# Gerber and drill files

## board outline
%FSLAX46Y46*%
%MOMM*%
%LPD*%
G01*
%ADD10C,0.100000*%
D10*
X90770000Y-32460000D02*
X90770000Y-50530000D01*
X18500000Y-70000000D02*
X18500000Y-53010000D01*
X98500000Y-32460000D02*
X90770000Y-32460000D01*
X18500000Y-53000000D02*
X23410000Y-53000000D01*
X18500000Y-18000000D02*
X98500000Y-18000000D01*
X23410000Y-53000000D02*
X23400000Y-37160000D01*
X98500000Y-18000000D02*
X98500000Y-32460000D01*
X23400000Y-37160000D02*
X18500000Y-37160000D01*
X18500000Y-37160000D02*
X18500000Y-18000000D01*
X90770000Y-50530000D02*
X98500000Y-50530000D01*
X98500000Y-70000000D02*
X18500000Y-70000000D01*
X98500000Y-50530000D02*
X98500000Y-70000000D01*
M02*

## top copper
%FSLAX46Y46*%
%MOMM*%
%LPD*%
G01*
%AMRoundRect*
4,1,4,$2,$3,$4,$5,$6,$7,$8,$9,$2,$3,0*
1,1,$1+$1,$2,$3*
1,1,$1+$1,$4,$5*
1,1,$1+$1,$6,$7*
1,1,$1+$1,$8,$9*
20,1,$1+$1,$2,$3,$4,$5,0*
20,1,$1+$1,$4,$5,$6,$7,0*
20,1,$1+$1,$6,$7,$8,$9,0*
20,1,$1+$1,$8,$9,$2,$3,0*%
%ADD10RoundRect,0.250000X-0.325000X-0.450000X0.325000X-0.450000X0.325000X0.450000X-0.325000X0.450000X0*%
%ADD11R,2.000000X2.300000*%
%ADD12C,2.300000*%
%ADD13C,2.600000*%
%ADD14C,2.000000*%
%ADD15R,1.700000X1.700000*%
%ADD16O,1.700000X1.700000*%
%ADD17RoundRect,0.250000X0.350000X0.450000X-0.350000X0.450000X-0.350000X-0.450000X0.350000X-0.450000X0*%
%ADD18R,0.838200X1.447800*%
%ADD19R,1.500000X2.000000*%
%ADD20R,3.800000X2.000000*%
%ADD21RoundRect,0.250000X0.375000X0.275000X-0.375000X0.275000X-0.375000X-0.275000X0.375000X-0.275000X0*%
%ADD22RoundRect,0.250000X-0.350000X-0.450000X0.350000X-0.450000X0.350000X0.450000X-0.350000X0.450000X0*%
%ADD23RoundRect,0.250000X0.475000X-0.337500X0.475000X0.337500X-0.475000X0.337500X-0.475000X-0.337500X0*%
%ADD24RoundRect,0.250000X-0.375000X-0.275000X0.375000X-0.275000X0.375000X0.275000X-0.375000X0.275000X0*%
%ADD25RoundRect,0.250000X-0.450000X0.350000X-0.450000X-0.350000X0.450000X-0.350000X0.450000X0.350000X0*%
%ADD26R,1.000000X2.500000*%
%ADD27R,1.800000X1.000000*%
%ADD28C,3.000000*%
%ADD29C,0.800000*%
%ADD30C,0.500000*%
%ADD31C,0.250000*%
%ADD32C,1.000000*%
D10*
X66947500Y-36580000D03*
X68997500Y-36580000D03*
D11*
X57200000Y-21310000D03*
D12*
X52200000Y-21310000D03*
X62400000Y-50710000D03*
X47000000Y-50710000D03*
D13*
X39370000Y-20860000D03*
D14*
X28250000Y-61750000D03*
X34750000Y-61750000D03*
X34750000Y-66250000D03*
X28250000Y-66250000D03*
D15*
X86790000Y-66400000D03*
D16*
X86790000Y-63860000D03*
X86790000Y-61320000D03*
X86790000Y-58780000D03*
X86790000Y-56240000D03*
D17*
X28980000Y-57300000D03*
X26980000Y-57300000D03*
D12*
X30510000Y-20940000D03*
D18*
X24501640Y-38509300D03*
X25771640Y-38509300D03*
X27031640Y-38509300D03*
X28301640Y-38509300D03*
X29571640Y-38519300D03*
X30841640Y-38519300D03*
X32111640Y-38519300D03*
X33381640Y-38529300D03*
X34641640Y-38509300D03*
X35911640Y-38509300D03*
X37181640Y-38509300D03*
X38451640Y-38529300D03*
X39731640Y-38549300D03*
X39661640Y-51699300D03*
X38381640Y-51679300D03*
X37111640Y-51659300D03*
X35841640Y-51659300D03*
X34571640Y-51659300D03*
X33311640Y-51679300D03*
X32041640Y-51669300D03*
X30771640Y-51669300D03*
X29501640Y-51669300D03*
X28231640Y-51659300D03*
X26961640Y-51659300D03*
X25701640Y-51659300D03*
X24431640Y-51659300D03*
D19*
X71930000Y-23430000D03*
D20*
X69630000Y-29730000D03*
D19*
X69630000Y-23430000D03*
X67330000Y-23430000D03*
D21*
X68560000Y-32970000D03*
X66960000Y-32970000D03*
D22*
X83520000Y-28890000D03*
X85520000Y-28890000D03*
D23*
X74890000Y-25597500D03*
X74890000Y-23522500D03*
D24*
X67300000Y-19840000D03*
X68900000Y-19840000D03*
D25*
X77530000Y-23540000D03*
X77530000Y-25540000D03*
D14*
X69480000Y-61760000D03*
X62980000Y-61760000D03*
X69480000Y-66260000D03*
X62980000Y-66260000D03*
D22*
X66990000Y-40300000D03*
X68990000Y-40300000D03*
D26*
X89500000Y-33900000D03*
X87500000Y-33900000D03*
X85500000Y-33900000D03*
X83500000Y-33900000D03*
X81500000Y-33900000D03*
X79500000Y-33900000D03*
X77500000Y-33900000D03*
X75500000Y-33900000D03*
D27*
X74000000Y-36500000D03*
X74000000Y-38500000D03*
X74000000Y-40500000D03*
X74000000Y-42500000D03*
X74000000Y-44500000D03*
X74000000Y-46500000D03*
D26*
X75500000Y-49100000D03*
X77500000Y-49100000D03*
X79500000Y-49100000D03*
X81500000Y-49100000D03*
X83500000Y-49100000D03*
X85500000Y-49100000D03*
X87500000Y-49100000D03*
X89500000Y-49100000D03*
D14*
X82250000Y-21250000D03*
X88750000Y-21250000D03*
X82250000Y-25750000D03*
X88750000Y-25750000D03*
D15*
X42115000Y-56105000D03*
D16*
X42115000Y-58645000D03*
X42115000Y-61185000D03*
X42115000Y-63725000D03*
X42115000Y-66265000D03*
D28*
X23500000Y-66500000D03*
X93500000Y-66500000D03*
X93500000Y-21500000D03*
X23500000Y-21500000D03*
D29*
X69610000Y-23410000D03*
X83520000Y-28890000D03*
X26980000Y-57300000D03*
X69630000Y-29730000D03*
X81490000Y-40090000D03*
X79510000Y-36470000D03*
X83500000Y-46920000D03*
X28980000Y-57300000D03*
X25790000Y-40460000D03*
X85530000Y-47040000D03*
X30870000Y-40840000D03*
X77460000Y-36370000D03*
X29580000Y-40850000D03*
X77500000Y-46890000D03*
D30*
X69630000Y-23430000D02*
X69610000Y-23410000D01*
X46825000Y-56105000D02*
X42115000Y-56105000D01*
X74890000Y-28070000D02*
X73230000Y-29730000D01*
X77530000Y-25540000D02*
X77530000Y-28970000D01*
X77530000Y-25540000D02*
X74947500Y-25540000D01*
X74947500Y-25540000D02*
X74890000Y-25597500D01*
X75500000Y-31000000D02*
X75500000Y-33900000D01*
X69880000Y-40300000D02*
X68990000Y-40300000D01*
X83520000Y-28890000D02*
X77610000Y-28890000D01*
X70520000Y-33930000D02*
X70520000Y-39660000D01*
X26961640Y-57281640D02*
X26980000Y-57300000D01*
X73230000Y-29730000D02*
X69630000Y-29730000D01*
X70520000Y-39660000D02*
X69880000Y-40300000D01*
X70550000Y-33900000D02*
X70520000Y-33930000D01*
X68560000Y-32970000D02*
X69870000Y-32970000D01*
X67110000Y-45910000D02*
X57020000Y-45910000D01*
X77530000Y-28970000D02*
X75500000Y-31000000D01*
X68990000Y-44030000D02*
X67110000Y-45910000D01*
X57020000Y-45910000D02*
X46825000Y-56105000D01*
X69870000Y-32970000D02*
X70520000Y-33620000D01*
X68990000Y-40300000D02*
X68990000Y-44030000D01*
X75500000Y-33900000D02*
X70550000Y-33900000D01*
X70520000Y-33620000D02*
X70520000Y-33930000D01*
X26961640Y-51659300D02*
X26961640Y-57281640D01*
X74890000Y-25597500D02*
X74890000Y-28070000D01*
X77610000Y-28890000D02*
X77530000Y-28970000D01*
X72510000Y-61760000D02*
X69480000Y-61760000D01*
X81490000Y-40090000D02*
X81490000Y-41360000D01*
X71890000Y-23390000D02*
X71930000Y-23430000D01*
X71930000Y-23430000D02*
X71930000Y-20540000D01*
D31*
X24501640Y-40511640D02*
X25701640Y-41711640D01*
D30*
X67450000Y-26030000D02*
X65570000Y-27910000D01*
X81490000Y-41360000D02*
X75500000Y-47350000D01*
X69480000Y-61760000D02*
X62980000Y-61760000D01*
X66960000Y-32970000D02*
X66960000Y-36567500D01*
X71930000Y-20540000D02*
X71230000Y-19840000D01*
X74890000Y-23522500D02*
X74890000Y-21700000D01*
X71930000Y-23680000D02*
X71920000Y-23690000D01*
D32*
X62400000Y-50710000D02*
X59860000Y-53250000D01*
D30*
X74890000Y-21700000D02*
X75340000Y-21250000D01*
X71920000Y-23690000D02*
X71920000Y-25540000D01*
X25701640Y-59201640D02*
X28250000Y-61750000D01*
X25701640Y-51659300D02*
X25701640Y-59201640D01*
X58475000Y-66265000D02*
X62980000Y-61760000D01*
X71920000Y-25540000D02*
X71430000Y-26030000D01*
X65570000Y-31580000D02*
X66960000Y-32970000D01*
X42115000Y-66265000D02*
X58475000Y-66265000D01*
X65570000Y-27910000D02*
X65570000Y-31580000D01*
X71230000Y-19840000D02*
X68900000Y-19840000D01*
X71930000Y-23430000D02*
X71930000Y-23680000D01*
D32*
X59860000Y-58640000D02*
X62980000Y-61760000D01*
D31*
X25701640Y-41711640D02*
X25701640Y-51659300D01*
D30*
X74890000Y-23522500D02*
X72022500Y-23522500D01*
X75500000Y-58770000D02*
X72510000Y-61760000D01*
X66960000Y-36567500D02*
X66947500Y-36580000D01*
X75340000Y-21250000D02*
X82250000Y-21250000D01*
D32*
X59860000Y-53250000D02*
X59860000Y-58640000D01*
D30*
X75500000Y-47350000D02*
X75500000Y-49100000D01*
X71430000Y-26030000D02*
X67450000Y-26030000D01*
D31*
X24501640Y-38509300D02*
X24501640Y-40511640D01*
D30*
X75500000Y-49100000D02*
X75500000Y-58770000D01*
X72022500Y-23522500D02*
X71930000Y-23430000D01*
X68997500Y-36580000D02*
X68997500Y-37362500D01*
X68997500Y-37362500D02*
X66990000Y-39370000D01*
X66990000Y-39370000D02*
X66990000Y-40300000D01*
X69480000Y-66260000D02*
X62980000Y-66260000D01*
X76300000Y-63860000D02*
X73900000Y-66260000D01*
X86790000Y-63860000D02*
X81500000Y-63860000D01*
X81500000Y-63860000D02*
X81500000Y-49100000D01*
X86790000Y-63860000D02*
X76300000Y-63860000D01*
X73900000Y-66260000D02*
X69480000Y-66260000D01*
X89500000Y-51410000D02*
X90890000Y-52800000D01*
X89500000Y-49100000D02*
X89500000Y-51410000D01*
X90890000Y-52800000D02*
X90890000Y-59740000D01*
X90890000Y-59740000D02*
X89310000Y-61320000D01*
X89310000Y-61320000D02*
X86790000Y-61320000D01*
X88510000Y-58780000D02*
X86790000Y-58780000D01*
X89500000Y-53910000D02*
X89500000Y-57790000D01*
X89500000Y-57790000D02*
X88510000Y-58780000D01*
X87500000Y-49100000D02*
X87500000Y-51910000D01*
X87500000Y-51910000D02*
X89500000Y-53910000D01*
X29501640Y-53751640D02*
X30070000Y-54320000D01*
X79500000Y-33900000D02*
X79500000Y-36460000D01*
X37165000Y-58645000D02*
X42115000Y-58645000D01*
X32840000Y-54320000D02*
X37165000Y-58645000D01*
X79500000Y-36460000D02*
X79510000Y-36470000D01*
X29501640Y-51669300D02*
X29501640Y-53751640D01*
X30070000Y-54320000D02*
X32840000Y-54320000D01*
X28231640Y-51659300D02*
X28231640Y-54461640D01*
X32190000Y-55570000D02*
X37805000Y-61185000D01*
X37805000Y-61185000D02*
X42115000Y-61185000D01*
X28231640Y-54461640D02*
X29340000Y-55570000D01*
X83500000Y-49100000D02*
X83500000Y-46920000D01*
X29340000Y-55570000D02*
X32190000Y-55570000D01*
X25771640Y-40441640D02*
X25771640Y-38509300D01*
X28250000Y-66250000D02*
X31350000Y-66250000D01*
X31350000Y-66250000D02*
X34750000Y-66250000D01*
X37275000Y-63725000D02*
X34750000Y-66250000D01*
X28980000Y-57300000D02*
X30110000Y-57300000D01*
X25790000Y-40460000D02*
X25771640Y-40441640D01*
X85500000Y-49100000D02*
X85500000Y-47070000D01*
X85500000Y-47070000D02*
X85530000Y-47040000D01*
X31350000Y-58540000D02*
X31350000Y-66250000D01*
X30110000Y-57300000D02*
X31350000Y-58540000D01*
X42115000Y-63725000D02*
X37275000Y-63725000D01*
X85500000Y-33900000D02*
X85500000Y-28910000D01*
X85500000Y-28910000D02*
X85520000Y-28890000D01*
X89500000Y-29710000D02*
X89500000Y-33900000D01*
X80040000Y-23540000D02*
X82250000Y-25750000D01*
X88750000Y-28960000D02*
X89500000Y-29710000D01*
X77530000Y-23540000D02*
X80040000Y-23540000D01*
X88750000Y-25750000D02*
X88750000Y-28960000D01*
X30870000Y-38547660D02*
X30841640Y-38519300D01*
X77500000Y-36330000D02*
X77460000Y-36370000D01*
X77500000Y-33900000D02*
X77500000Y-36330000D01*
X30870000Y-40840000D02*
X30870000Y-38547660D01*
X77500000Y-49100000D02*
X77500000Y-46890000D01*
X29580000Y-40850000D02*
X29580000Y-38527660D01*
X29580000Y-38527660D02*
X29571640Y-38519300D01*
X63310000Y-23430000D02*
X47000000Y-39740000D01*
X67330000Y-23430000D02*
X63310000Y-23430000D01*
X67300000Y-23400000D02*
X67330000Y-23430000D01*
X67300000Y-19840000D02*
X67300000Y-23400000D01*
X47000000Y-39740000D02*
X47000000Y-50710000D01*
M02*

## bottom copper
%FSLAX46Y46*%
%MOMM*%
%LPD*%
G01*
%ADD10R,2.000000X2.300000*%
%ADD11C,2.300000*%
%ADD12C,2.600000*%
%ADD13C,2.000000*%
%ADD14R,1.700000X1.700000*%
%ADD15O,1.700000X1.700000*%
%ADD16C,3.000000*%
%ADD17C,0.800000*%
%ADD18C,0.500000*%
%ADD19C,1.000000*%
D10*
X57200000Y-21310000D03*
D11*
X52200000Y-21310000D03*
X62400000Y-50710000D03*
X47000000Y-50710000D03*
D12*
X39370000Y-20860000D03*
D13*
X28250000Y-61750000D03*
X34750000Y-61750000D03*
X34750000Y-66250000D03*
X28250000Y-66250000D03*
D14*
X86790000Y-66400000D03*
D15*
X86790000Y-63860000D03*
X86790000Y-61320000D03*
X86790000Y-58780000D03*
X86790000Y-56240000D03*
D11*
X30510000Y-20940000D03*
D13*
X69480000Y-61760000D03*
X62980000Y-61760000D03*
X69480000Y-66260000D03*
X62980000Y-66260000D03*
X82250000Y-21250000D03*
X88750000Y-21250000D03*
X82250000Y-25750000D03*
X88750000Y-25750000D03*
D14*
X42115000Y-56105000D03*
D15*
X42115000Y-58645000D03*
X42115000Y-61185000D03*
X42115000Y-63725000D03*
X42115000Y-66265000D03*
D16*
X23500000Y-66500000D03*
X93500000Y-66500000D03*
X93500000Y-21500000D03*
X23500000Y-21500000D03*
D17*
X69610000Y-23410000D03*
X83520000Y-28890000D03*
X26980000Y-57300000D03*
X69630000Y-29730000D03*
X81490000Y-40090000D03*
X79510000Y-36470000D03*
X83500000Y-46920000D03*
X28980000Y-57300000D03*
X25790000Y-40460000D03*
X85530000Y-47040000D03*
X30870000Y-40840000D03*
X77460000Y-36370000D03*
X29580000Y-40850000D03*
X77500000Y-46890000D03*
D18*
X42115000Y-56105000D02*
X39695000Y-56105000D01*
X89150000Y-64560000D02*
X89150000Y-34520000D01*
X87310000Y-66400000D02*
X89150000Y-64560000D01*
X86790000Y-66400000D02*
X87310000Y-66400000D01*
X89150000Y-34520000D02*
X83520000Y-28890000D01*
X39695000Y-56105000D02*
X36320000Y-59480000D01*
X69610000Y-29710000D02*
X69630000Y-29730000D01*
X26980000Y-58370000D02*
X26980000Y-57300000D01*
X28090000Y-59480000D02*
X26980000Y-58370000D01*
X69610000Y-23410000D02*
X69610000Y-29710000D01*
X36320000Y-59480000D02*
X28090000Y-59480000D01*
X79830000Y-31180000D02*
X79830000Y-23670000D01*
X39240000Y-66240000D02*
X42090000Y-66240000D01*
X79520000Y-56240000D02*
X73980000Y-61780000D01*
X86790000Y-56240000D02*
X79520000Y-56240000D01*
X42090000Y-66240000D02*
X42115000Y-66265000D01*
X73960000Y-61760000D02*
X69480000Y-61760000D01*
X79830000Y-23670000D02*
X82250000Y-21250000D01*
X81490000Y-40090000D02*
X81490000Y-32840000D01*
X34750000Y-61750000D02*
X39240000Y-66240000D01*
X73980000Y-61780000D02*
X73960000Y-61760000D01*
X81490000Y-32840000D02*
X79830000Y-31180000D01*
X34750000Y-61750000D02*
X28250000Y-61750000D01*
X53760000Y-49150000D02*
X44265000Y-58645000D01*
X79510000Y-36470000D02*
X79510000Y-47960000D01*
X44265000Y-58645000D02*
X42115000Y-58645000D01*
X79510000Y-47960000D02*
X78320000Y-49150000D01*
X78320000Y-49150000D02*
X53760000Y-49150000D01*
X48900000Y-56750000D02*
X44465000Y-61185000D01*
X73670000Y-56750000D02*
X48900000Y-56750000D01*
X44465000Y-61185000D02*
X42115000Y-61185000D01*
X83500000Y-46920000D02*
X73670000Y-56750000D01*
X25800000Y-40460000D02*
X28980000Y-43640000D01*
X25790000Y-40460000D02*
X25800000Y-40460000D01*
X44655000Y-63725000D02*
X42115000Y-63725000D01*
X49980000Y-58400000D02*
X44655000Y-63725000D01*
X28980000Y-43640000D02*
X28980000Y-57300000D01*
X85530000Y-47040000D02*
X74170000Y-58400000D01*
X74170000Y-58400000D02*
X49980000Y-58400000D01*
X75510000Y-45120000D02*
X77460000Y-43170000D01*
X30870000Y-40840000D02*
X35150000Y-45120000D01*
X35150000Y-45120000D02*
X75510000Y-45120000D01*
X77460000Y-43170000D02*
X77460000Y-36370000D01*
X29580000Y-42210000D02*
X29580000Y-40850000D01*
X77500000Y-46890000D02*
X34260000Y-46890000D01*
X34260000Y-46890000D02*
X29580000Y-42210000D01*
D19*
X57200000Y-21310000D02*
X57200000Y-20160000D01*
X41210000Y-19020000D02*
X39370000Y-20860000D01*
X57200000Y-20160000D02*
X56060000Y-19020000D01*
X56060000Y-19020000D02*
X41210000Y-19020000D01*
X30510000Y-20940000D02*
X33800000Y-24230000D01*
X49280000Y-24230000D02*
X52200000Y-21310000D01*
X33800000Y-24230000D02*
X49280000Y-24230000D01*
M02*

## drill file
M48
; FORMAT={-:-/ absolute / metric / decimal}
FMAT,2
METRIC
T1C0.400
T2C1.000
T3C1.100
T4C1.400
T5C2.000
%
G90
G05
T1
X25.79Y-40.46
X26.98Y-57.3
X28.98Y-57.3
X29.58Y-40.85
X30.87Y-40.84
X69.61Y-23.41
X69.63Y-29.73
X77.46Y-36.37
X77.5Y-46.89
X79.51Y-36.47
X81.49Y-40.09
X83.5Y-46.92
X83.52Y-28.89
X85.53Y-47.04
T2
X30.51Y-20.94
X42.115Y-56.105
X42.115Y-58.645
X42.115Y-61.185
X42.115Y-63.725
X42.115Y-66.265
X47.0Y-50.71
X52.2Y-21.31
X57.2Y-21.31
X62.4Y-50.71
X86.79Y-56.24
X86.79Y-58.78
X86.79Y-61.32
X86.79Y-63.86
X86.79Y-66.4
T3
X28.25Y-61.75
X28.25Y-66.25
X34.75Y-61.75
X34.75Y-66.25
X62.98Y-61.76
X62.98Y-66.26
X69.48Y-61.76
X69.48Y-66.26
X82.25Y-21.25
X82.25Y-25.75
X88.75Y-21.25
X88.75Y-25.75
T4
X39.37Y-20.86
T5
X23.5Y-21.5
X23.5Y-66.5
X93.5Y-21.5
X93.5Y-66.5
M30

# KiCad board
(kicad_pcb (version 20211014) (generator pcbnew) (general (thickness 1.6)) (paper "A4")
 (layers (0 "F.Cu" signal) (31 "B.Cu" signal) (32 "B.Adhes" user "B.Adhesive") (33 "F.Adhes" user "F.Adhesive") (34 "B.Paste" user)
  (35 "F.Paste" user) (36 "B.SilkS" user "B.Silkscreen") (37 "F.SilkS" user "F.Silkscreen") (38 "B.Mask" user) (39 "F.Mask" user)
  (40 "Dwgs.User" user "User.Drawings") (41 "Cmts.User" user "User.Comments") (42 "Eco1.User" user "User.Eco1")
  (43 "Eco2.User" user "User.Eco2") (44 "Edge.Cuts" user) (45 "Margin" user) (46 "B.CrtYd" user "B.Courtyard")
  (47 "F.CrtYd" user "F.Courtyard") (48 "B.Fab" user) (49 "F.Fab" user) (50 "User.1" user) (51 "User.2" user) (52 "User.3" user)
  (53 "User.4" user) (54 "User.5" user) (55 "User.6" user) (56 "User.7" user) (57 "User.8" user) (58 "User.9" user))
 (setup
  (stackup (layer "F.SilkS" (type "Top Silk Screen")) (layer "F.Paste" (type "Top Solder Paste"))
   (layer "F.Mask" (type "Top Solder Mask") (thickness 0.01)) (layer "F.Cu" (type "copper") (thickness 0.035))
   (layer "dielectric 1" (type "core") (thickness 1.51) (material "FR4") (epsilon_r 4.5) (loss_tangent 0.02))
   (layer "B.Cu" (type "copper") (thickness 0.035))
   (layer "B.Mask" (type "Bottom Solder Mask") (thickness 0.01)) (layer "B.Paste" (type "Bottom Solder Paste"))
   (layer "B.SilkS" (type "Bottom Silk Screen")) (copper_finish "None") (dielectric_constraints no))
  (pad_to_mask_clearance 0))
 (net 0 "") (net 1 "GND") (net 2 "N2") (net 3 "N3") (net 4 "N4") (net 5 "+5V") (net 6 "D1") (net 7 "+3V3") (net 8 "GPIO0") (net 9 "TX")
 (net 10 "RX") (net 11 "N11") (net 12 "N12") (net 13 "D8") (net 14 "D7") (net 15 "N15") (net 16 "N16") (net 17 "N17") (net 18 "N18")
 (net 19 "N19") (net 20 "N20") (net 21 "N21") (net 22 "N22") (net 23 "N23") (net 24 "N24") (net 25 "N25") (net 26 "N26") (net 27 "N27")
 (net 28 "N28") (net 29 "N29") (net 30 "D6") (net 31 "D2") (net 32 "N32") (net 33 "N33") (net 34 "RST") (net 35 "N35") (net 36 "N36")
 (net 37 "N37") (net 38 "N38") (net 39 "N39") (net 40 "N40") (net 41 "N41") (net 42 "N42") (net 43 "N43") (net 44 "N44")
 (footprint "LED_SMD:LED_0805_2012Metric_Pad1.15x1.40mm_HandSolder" (layer "F.Cu") (at 67.9725 36.58)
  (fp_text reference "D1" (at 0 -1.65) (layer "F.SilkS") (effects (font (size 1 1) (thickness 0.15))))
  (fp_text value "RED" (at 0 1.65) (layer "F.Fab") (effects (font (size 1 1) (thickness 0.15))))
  (pad "1" smd roundrect (at -1.025 0) (size 1.15 1.4) (layers "F.Cu" "F.Paste" "F.Mask") (roundrect_rratio 0.217391) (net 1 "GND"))
  (pad "2" smd roundrect (at 1.025 0) (size 1.15 1.4) (layers "F.Cu" "F.Paste" "F.Mask") (roundrect_rratio 0.217391) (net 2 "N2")))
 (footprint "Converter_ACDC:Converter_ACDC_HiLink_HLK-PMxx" (layer "F.Cu") (at 57.2 21.31 -90)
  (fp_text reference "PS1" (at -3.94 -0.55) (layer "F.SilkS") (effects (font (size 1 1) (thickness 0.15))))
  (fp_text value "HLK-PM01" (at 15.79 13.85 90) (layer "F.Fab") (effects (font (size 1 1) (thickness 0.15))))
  (pad "1" thru_hole rect (at 0 0 270) (size 2.3 2) (drill 1) (layers *.Cu *.Mask) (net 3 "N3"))
  (pad "2" thru_hole circle (at 0 5 270) (size 2.3 2.3) (drill 1) (layers *.Cu *.Mask) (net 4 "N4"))
  (pad "3" thru_hole circle (at 29.4 -5.2 270) (size 2.3 2.3) (drill 1) (layers *.Cu *.Mask) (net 1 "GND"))
  (pad "4" thru_hole circle (at 29.4 10.2 270) (size 2.3 2.3) (drill 1) (layers *.Cu *.Mask) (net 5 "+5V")))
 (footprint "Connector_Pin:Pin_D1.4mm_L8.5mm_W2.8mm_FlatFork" (layer "F.Cu") (at 39.37 20.86)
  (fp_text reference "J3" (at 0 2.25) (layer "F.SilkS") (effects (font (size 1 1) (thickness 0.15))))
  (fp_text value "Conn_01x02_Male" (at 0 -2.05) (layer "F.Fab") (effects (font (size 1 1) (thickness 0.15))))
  (pad "1" thru_hole circle (at 0 0) (size 2.6 2.6) (drill 1.4) (layers *.Cu *.Mask) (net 3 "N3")))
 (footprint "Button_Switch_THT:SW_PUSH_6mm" (layer "F.Cu") (at 28.25 61.75)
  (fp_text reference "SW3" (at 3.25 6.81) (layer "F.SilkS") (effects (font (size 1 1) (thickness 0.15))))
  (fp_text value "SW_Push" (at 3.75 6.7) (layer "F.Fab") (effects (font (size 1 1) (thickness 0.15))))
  (pad "1" thru_hole circle (at 0 0 90) (size 2 2) (drill 1.1) (layers *.Cu *.Mask) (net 1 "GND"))
  (pad "1" thru_hole circle (at 6.5 0 90) (size 2 2) (drill 1.1) (layers *.Cu *.Mask) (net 1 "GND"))
  (pad "2" thru_hole circle (at 6.5 4.5 90) (size 2 2) (drill 1.1) (layers *.Cu *.Mask) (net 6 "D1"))
  (pad "2" thru_hole circle (at 0 4.5 90) (size 2 2) (drill 1.1) (layers *.Cu *.Mask) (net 6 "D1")))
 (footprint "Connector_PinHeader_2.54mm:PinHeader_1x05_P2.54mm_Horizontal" (layer "F.Cu") (at 86.79 66.4 180)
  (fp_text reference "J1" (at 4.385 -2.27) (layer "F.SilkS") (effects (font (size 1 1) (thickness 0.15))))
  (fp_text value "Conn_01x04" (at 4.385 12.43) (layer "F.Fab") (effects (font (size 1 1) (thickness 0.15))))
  (pad "1" thru_hole rect (at 0 0 180) (size 1.7 1.7) (drill 1) (layers *.Cu *.Mask) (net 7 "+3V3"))
  (pad "2" thru_hole oval (at 0 2.54 180) (size 1.7 1.7) (drill 1) (layers *.Cu *.Mask) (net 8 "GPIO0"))
  (pad "3" thru_hole oval (at 0 5.08 180) (size 1.7 1.7) (drill 1) (layers *.Cu *.Mask) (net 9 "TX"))
  (pad "4" thru_hole oval (at 0 7.62 180) (size 1.7 1.7) (drill 1) (layers *.Cu *.Mask) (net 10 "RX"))
  (pad "5" thru_hole oval (at 0 10.16 180) (size 1.7 1.7) (drill 1) (layers *.Cu *.Mask) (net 1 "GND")))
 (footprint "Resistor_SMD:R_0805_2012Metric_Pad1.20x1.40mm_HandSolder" (layer "F.Cu") (at 27.98 57.3 180)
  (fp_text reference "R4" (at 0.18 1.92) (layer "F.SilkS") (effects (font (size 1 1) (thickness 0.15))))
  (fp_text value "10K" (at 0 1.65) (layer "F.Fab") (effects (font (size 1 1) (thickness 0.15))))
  (pad "1" smd roundrect (at -1 0 180) (size 1.2 1.4) (layers "F.Cu" "F.Paste" "F.Mask") (roundrect_rratio 0.208333) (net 6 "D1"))
  (pad "2" smd roundrect (at 1 0 180) (size 1.2 1.4) (layers "F.Cu" "F.Paste" "F.Mask") (roundrect_rratio 0.208333) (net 7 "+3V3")))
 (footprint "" (layer "F.Cu") (at 30.51 20.94)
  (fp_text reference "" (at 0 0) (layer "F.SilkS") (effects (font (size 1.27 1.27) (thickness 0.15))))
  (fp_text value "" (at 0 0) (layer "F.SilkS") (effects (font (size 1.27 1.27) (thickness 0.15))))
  (pad "2" thru_hole circle (at 0 0 270) (size 2.3 2.3) (drill 1) (layers *.Cu *.Mask) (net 4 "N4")))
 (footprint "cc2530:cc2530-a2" (layer "F.Cu") (at 29.09396 45.0625 90)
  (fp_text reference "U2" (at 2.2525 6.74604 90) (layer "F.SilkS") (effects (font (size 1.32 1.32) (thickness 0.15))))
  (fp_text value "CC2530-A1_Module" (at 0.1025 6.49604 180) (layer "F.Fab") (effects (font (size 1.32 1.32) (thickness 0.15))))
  (pad "1" smd rect (at 6.5532 -4.59232 90) (size 1.4478 0.8382) (layers "F.Cu" "F.Paste" "F.Mask") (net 1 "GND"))
  (pad "2" smd rect (at 6.5532 -3.32232 90) (size 1.4478 0.8382) (layers "F.Cu" "F.Paste" "F.Mask") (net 6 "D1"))
  (pad "3" smd rect (at 6.5532 -2.06232 90) (size 1.4478 0.8382) (layers "F.Cu" "F.Paste" "F.Mask") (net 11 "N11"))
  (pad "4" smd rect (at 6.5532 -0.79232 90) (size 1.4478 0.8382) (layers "F.Cu" "F.Paste" "F.Mask") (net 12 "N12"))
  (pad "5" smd rect (at 6.5432 0.47768 90) (size 1.4478 0.8382) (layers "F.Cu" "F.Paste" "F.Mask") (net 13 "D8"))
  (pad "6" smd rect (at 6.5432 1.74768 90) (size 1.4478 0.8382) (layers "F.Cu" "F.Paste" "F.Mask") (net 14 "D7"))
  (pad "7" smd rect (at 6.5432 3.01768 90) (size 1.4478 0.8382) (layers "F.Cu" "F.Paste" "F.Mask") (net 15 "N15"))
  (pad "8" smd rect (at 6.5332 4.28768 90) (size 1.4478 0.8382) (layers "F.Cu" "F.Paste" "F.Mask") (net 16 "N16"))
  (pad "9" smd rect (at 6.5532 5.54768 90) (size 1.4478 0.8382) (layers "F.Cu" "F.Paste" "F.Mask") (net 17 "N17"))
  (pad "10" smd rect (at 6.5532 6.81768 90) (size 1.4478 0.8382) (layers "F.Cu" "F.Paste" "F.Mask") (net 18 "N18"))
  (pad "11" smd rect (at 6.5532 8.08768 90) (size 1.4478 0.8382) (layers "F.Cu" "F.Paste" "F.Mask") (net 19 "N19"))
  (pad "12" smd rect (at 6.5332 9.35768 90) (size 1.4478 0.8382) (layers "F.Cu" "F.Paste" "F.Mask") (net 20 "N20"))
  (pad "13" smd rect (at 6.5132 10.63768 270) (size 1.4478 0.8382) (layers "F.Cu" "F.Paste" "F.Mask") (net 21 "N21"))
  (pad "14" smd rect (at -6.6368 10.56768 270) (size 1.4478 0.8382) (layers "F.Cu" "F.Paste" "F.Mask") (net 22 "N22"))
  (pad "15" smd rect (at -6.6168 9.28768 90) (size 1.4478 0.8382) (layers "F.Cu" "F.Paste" "F.Mask") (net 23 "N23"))
  (pad "16" smd rect (at -6.5968 8.01768 90) (size 1.4478 0.8382) (layers "F.Cu" "F.Paste" "F.Mask") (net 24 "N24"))
  (pad "17" smd rect (at -6.5968 6.74768 90) (size 1.4478 0.8382) (layers "F.Cu" "F.Paste" "F.Mask") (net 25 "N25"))
  (pad "18" smd rect (at -6.5968 5.47768 90) (size 1.4478 0.8382) (layers "F.Cu" "F.Paste" "F.Mask") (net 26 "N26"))
  (pad "19" smd rect (at -6.6168 4.21768 90) (size 1.4478 0.8382) (layers "F.Cu" "F.Paste" "F.Mask") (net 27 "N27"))
  (pad "20" smd rect (at -6.6068 2.94768 90) (size 1.4478 0.8382) (layers "F.Cu" "F.Paste" "F.Mask") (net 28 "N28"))
  (pad "21" smd rect (at -6.6068 1.67768 90) (size 1.4478 0.8382) (layers "F.Cu" "F.Paste" "F.Mask") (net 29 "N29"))
  (pad "22" smd rect (at -6.6068 0.40768 90) (size 1.4478 0.8382) (layers "F.Cu" "F.Paste" "F.Mask") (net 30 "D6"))
  (pad "23" smd rect (at -6.5968 -0.86232 90) (size 1.4478 0.8382) (layers "F.Cu" "F.Paste" "F.Mask") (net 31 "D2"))
  (pad "24" smd rect (at -6.5968 -2.13232 90) (size 1.4478 0.8382) (layers "F.Cu" "F.Paste" "F.Mask") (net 7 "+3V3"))
  (pad "25" smd rect (at -6.5968 -3.39232 90) (size 1.4478 0.8382) (layers "F.Cu" "F.Paste" "F.Mask") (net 1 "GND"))
  (pad "26" smd rect (at -6.5968 -4.66232 90) (size 1.4478 0.8382) (layers "F.Cu" "F.Paste" "F.Mask") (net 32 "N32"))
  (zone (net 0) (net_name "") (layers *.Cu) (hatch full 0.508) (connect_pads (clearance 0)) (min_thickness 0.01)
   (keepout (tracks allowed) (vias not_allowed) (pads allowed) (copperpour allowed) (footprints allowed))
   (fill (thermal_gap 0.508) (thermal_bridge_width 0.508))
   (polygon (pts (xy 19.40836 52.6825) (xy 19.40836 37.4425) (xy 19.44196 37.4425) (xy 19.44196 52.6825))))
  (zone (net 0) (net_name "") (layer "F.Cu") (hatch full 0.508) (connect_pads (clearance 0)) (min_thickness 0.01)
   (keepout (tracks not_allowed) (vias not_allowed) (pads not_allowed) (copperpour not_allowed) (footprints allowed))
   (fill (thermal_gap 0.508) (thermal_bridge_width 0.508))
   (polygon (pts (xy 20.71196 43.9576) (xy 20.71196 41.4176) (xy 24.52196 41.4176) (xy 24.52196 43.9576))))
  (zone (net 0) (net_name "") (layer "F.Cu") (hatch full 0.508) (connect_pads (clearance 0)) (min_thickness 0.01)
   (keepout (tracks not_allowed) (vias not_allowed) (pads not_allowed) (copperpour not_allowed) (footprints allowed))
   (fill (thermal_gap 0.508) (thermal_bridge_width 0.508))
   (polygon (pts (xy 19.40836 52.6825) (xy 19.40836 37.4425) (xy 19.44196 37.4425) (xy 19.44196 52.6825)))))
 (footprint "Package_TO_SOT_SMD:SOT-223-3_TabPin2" (layer "F.Cu") (at 69.63 26.58 -90)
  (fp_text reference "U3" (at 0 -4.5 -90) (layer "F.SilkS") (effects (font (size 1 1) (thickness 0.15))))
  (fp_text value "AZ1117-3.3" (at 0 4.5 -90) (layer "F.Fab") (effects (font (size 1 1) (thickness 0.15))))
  (pad "1" smd rect (at -3.15 -2.3 270) (size 2 1.5) (layers "F.Cu" "F.Paste" "F.Mask") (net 1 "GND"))
  (pad "2" smd rect (at 3.15 0 270) (size 2 3.8) (layers "F.Cu" "F.Paste" "F.Mask") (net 7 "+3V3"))
  (pad "2" smd rect (at -3.15 0 270) (size 2 1.5) (layers "F.Cu" "F.Paste" "F.Mask") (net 7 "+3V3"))
  (pad "3" smd rect (at -3.15 2.3 270) (size 2 1.5) (layers "F.Cu" "F.Paste" "F.Mask") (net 5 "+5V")))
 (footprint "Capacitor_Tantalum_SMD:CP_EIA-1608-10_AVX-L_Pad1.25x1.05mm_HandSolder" (layer "F.Cu") (at 67.76 32.97 180)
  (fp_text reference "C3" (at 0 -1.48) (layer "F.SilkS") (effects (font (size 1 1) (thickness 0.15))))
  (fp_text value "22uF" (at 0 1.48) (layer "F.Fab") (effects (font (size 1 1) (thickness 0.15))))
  (pad "1" smd roundrect (at -0.8 0 180) (size 1.25 1.05) (layers "F.Cu" "F.Paste" "F.Mask") (roundrect_rratio 0.238095) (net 7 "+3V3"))
  (pad "2" smd roundrect (at 0.8 0 180) (size 1.25 1.05) (layers "F.Cu" "F.Paste" "F.Mask") (roundrect_rratio 0.238095) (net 1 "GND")))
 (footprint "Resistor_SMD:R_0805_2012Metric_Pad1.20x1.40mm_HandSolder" (layer "F.Cu") (at 84.52 28.89)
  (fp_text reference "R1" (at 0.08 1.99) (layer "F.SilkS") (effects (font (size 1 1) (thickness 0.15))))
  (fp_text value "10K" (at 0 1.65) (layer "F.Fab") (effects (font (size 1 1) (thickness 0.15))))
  (pad "1" smd roundrect (at -1 0) (size 1.2 1.4) (layers "F.Cu" "F.Paste" "F.Mask") (roundrect_rratio 0.208333) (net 7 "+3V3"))
  (pad "2" smd roundrect (at 1 0) (size 1.2 1.4) (layers "F.Cu" "F.Paste" "F.Mask") (roundrect_rratio 0.208333) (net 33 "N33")))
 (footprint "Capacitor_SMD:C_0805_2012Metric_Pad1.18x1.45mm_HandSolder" (layer "F.Cu") (at 74.89 24.56 90)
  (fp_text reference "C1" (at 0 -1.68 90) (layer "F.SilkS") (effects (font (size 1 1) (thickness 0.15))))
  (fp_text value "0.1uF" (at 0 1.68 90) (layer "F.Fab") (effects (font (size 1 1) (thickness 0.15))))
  (pad "1" smd roundrect (at -1.0375 0 90) (size 1.175 1.45) (layers "F.Cu" "F.Paste" "F.Mask") (roundrect_rratio 0.212766) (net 7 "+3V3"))
  (pad "2" smd roundrect (at 1.0375 0 90) (size 1.175 1.45) (layers "F.Cu" "F.Paste" "F.Mask") (roundrect_rratio 0.212766) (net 1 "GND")))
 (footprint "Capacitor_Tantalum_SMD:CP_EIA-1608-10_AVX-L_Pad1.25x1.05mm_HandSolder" (layer "F.Cu") (at 68.1 19.84)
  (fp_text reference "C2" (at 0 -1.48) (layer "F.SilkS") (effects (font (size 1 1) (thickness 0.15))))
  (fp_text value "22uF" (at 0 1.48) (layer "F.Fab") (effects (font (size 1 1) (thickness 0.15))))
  (pad "1" smd roundrect (at -0.8 0) (size 1.25 1.05) (layers "F.Cu" "F.Paste" "F.Mask") (roundrect_rratio 0.238095) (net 5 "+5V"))
  (pad "2" smd roundrect (at 0.8 0) (size 1.25 1.05) (layers "F.Cu" "F.Paste" "F.Mask") (roundrect_rratio 0.238095) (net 1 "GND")))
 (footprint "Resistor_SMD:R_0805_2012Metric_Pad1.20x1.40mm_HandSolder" (layer "F.Cu") (at 77.53 24.54 -90)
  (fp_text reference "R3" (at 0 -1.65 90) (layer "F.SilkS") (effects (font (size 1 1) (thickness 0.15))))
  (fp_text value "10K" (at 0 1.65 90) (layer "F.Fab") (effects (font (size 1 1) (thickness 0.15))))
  (pad "1" smd roundrect (at -1 0 270) (size 1.2 1.4) (layers "F.Cu" "F.Paste" "F.Mask") (roundrect_rratio 0.208333) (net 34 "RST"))
  (pad "2" smd roundrect (at 1 0 270) (size 1.2 1.4) (layers "F.Cu" "F.Paste" "F.Mask") (roundrect_rratio 0.208333) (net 7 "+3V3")))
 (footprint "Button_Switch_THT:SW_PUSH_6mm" (layer "F.Cu") (at 62.98 61.76)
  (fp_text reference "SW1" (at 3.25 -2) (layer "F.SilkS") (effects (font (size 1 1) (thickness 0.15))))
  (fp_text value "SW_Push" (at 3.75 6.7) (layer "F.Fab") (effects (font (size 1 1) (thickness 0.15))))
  (pad "1" thru_hole circle (at 6.5 0 90) (size 2 2) (drill 1.1) (layers *.Cu *.Mask) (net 1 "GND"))
  (pad "1" thru_hole circle (at 0 0 90) (size 2 2) (drill 1.1) (layers *.Cu *.Mask) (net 1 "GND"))
  (pad "2" thru_hole circle (at 6.5 4.5 90) (size 2 2) (drill 1.1) (layers *.Cu *.Mask) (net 8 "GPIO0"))
  (pad "2" thru_hole circle (at 0 4.5 90) (size 2 2) (drill 1.1) (layers *.Cu *.Mask) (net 8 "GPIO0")))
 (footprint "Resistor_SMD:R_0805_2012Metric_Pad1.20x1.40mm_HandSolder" (layer "F.Cu") (at 67.99 40.3)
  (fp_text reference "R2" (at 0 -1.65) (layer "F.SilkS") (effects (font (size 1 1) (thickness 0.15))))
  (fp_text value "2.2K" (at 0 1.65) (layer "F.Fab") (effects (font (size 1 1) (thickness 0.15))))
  (pad "1" smd roundrect (at -1 0) (size 1.2 1.4) (layers "F.Cu" "F.Paste" "F.Mask") (roundrect_rratio 0.208333) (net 2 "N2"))
  (pad "2" smd roundrect (at 1 0) (size 1.2 1.4) (layers "F.Cu" "F.Paste" "F.Mask") (roundrect_rratio 0.208333) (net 7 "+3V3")))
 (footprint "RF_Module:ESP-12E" (layer "F.Cu") (at 86 41.5 -90)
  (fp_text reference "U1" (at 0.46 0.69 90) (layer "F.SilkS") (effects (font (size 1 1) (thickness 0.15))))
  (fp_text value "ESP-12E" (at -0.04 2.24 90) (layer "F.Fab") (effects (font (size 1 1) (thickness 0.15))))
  (pad "1" smd rect (at -7.6 -3.5 270) (size 2.5 1) (layers "F.Cu" "F.Paste" "F.Mask") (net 34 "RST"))
  (pad "2" smd rect (at -7.6 -1.5 270) (size 2.5 1) (layers "F.Cu" "F.Paste" "F.Mask") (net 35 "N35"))
  (pad "3" smd rect (at -7.6 0.5 270) (size 2.5 1) (layers "F.Cu" "F.Paste" "F.Mask") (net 33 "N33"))
  (pad "4" smd rect (at -7.6 2.5 270) (size 2.5 1) (layers "F.Cu" "F.Paste" "F.Mask") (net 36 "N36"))
  (pad "5" smd rect (at -7.6 4.5 270) (size 2.5 1) (layers "F.Cu" "F.Paste" "F.Mask") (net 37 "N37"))
  (pad "6" smd rect (at -7.6 6.5 270) (size 2.5 1) (layers "F.Cu" "F.Paste" "F.Mask") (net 30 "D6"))
  (pad "7" smd rect (at -7.6 8.5 270) (size 2.5 1) (layers "F.Cu" "F.Paste" "F.Mask") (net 14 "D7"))
  (pad "8" smd rect (at -7.6 10.5 270) (size 2.5 1) (layers "F.Cu" "F.Paste" "F.Mask") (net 7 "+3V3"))
  (pad "9" smd rect (at -5 12 270) (size 1 1.8) (layers "F.Cu" "F.Paste" "F.Mask") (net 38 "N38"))
  (pad "10" smd rect (at -3 12 270) (size 1 1.8) (layers "F.Cu" "F.Paste" "F.Mask") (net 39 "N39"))
  (pad "11" smd rect (at -1 12 270) (size 1 1.8) (layers "F.Cu" "F.Paste" "F.Mask") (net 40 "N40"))
  (pad "12" smd rect (at 1 12 270) (size 1 1.8) (layers "F.Cu" "F.Paste" "F.Mask") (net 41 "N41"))
  (pad "13" smd rect (at 3 12 270) (size 1 1.8) (layers "F.Cu" "F.Paste" "F.Mask") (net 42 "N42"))
  (pad "14" smd rect (at 5 12 270) (size 1 1.8) (layers "F.Cu" "F.Paste" "F.Mask") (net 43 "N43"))
  (pad "15" smd rect (at 7.6 10.5 270) (size 2.5 1) (layers "F.Cu" "F.Paste" "F.Mask") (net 1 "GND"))
  (pad "16" smd rect (at 7.6 8.5 270) (size 2.5 1) (layers "F.Cu" "F.Paste" "F.Mask") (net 13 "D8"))
  (pad "17" smd rect (at 7.6 6.5 270) (size 2.5 1) (layers "F.Cu" "F.Paste" "F.Mask") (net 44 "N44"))
  (pad "18" smd rect (at 7.6 4.5 270) (size 2.5 1) (layers "F.Cu" "F.Paste" "F.Mask") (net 8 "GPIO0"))
  (pad "19" smd rect (at 7.6 2.5 270) (size 2.5 1) (layers "F.Cu" "F.Paste" "F.Mask") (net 31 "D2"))
  (pad "20" smd rect (at 7.6 0.5 270) (size 2.5 1) (layers "F.Cu" "F.Paste" "F.Mask") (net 6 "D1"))
  (pad "21" smd rect (at 7.6 -1.5 270) (size 2.5 1) (layers "F.Cu" "F.Paste" "F.Mask") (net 10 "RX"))
  (pad "22" smd rect (at 7.6 -3.5 270) (size 2.5 1) (layers "F.Cu" "F.Paste" "F.Mask") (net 9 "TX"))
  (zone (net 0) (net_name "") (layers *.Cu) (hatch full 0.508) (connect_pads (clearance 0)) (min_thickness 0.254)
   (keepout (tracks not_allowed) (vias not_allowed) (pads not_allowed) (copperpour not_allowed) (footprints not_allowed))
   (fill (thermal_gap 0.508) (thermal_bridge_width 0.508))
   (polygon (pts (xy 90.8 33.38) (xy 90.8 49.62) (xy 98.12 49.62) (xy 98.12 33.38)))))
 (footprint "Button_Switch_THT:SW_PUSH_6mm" (layer "F.Cu") (at 82.25 21.25)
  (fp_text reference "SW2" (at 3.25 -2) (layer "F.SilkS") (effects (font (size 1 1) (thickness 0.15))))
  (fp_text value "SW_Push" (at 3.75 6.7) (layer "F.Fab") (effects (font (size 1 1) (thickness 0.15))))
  (pad "1" thru_hole circle (at 0 0 90) (size 2 2) (drill 1.1) (layers *.Cu *.Mask) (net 1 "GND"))
  (pad "1" thru_hole circle (at 6.5 0 90) (size 2 2) (drill 1.1) (layers *.Cu *.Mask) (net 1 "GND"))
  (pad "2" thru_hole circle (at 0 4.5 90) (size 2 2) (drill 1.1) (layers *.Cu *.Mask) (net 34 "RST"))
  (pad "2" thru_hole circle (at 6.5 4.5 90) (size 2 2) (drill 1.1) (layers *.Cu *.Mask) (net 34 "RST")))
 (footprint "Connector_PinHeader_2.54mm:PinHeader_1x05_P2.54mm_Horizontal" (layer "F.Cu") (at 42.115 56.105)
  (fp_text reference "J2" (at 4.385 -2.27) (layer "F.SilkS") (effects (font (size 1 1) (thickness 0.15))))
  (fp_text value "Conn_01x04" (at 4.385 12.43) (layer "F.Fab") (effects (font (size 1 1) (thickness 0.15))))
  (pad "1" thru_hole rect (at 0 0) (size 1.7 1.7) (drill 1) (layers *.Cu *.Mask) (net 7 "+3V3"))
  (pad "2" thru_hole oval (at 0 2.54) (size 1.7 1.7) (drill 1) (layers *.Cu *.Mask) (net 30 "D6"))
  (pad "3" thru_hole oval (at 0 5.08) (size 1.7 1.7) (drill 1) (layers *.Cu *.Mask) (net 31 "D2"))
  (pad "4" thru_hole oval (at 0 7.62) (size 1.7 1.7) (drill 1) (layers *.Cu *.Mask) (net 6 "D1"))
  (pad "5" thru_hole oval (at 0 10.16) (size 1.7 1.7) (drill 1) (layers *.Cu *.Mask) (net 1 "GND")))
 (gr_line (start 90.77 32.46) (end 90.77 50.53) (layer "Edge.Cuts") (width 0.1))
 (gr_line (start 18.5 70) (end 18.5 53.01) (layer "Edge.Cuts") (width 0.1))
 (gr_line (start 98.5 32.46) (end 90.77 32.46) (layer "Edge.Cuts") (width 0.1))
 (gr_line (start 18.5 53) (end 23.41 53) (layer "Edge.Cuts") (width 0.1))
 (gr_line (start 18.5 18) (end 98.5 18) (layer "Edge.Cuts") (width 0.1))
 (gr_line (start 23.41 53) (end 23.4 37.16) (layer "Edge.Cuts") (width 0.1))
 (gr_line (start 98.5 18) (end 98.5 32.46) (layer "Edge.Cuts") (width 0.1))
 (gr_line (start 23.4 37.16) (end 18.5 37.16) (layer "Edge.Cuts") (width 0.1))
 (gr_line (start 18.5 37.16) (end 18.5 18) (layer "Edge.Cuts") (width 0.1))
 (gr_line (start 90.77 50.53) (end 98.5 50.53) (layer "Edge.Cuts") (width 0.1))
 (gr_line (start 98.5 70) (end 18.5 70) (layer "Edge.Cuts") (width 0.1))
 (gr_line (start 98.5 50.53) (end 98.5 70) (layer "Edge.Cuts") (width 0.1))
 (via (at 23.5 66.5) (size 3) (drill 2) (layers "F.Cu" "B.Cu") (free) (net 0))
 (via (at 93.5 66.5) (size 3) (drill 2) (layers "F.Cu" "B.Cu") (free) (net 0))
 (via (at 93.5 21.5) (size 3) (drill 2) (layers "F.Cu" "B.Cu") (free) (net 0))
 (via (at 23.5 21.5) (size 3) (drill 2) (layers "F.Cu" "B.Cu") (free) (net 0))
 (segment (start 69.63 23.43) (end 69.61 23.41) (width 0.5) (layer "F.Cu") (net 7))
 (segment (start 46.825 56.105) (end 42.115 56.105) (width 0.5) (layer "F.Cu") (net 7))
 (segment (start 74.89 28.07) (end 73.23 29.73) (width 0.5) (layer "F.Cu") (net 7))
 (segment (start 77.53 25.54) (end 77.53 28.97) (width 0.5) (layer "F.Cu") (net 7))
 (segment (start 77.53 25.54) (end 74.9475 25.54) (width 0.5) (layer "F.Cu") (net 7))
 (segment (start 74.9475 25.54) (end 74.89 25.5975) (width 0.5) (layer "F.Cu") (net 7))
 (segment (start 75.5 31) (end 75.5 33.9) (width 0.5) (layer "F.Cu") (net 7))
 (segment (start 69.88 40.3) (end 68.99 40.3) (width 0.5) (layer "F.Cu") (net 7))
 (segment (start 83.52 28.89) (end 77.61 28.89) (width 0.5) (layer "F.Cu") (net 7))
 (segment (start 70.52 33.93) (end 70.52 39.66) (width 0.5) (layer "F.Cu") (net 7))
 (segment (start 26.96164 57.28164) (end 26.98 57.3) (width 0.5) (layer "F.Cu") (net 7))
 (segment (start 73.23 29.73) (end 69.63 29.73) (width 0.5) (layer "F.Cu") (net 7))
 (segment (start 70.52 39.66) (end 69.88 40.3) (width 0.5) (layer "F.Cu") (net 7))
 (segment (start 70.55 33.9) (end 70.52 33.93) (width 0.5) (layer "F.Cu") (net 7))
 (segment (start 68.56 32.97) (end 69.87 32.97) (width 0.5) (layer "F.Cu") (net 7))
 (segment (start 67.11 45.91) (end 57.02 45.91) (width 0.5) (layer "F.Cu") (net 7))
 (segment (start 77.53 28.97) (end 75.5 31) (width 0.5) (layer "F.Cu") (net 7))
 (segment (start 68.99 44.03) (end 67.11 45.91) (width 0.5) (layer "F.Cu") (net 7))
 (segment (start 57.02 45.91) (end 46.825 56.105) (width 0.5) (layer "F.Cu") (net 7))
 (segment (start 69.87 32.97) (end 70.52 33.62) (width 0.5) (layer "F.Cu") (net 7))
 (segment (start 68.99 40.3) (end 68.99 44.03) (width 0.5) (layer "F.Cu") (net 7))
 (segment (start 75.5 33.9) (end 70.55 33.9) (width 0.5) (layer "F.Cu") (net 7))
 (segment (start 70.52 33.62) (end 70.52 33.93) (width 0.5) (layer "F.Cu") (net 7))
 (segment (start 26.96164 51.6593) (end 26.96164 57.28164) (width 0.5) (layer "F.Cu") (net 7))
 (segment (start 74.89 25.5975) (end 74.89 28.07) (width 0.5) (layer "F.Cu") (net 7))
 (segment (start 77.61 28.89) (end 77.53 28.97) (width 0.5) (layer "F.Cu") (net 7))
 (via (at 69.61 23.41) (size 0.8) (drill 0.4) (layers "F.Cu" "B.Cu") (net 7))
 (via (at 83.52 28.89) (size 0.8) (drill 0.4) (layers "F.Cu" "B.Cu") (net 7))
 (via (at 26.98 57.3) (size 0.8) (drill 0.4) (layers "F.Cu" "B.Cu") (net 7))
 (via (at 69.63 29.73) (size 0.8) (drill 0.4) (layers "F.Cu" "B.Cu") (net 7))
 (segment (start 42.115 56.105) (end 39.695 56.105) (width 0.5) (layer "B.Cu") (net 7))
 (segment (start 89.15 64.56) (end 89.15 34.52) (width 0.5) (layer "B.Cu") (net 7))
 (segment (start 87.31 66.4) (end 89.15 64.56) (width 0.5) (layer "B.Cu") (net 7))
 (segment (start 86.79 66.4) (end 87.31 66.4) (width 0.5) (layer "B.Cu") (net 7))
 (segment (start 89.15 34.52) (end 83.52 28.89) (width 0.5) (layer "B.Cu") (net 7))
 (segment (start 39.695 56.105) (end 36.32 59.48) (width 0.5) (layer "B.Cu") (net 7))
 (segment (start 69.61 29.71) (end 69.63 29.73) (width 0.5) (layer "B.Cu") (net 7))
 (segment (start 26.98 58.37) (end 26.98 57.3) (width 0.5) (layer "B.Cu") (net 7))
 (segment (start 28.09 59.48) (end 26.98 58.37) (width 0.5) (layer "B.Cu") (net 7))
 (segment (start 69.61 23.41) (end 69.61 29.71) (width 0.5) (layer "B.Cu") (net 7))
 (segment (start 36.32 59.48) (end 28.09 59.48) (width 0.5) (layer "B.Cu") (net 7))
 (segment (start 72.51 61.76) (end 69.48 61.76) (width 0.5) (layer "F.Cu") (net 1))
 (segment (start 81.49 40.09) (end 81.49 41.36) (width 0.5) (layer "F.Cu") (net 1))
 (segment (start 71.89 23.39) (end 71.93 23.43) (width 0.5) (layer "F.Cu") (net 1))
 (segment (start 71.93 23.43) (end 71.93 20.54) (width 0.5) (layer "F.Cu") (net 1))
 (segment (start 24.50164 40.51164) (end 25.70164 41.71164) (width 0.25) (layer "F.Cu") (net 1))
 (segment (start 67.45 26.03) (end 65.57 27.91) (width 0.5) (layer "F.Cu") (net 1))
 (segment (start 81.49 41.36) (end 75.5 47.35) (width 0.5) (layer "F.Cu") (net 1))
 (segment (start 69.48 61.76) (end 62.98 61.76) (width 0.5) (layer "F.Cu") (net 1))
 (segment (start 66.96 32.97) (end 66.96 36.5675) (width 0.5) (layer "F.Cu") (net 1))
 (segment (start 71.93 20.54) (end 71.23 19.84) (width 0.5) (layer "F.Cu") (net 1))
 (segment (start 74.89 23.5225) (end 74.89 21.7) (width 0.5) (layer "F.Cu") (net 1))
 (segment (start 71.93 23.68) (end 71.92 23.69) (width 0.5) (layer "F.Cu") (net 1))
 (segment (start 62.4 50.71) (end 59.86 53.25) (width 1) (layer "F.Cu") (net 1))
 (segment (start 74.89 21.7) (end 75.34 21.25) (width 0.5) (layer "F.Cu") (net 1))
 (segment (start 71.92 23.69) (end 71.92 25.54) (width 0.5) (layer "F.Cu") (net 1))
 (segment (start 25.70164 59.20164) (end 28.25 61.75) (width 0.5) (layer "F.Cu") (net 1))
 (segment (start 25.70164 51.6593) (end 25.70164 59.20164) (width 0.5) (layer "F.Cu") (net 1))
 (segment (start 58.475 66.265) (end 62.98 61.76) (width 0.5) (layer "F.Cu") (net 1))
 (segment (start 71.92 25.54) (end 71.43 26.03) (width 0.5) (layer "F.Cu") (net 1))
 (segment (start 65.57 31.58) (end 66.96 32.97) (width 0.5) (layer "F.Cu") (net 1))
 (segment (start 42.115 66.265) (end 58.475 66.265) (width 0.5) (layer "F.Cu") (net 1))
 (segment (start 65.57 27.91) (end 65.57 31.58) (width 0.5) (layer "F.Cu") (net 1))
 (segment (start 71.23 19.84) (end 68.9 19.84) (width 0.5) (layer "F.Cu") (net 1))
 (segment (start 71.93 23.43) (end 71.93 23.68) (width 0.5) (layer "F.Cu") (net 1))
 (segment (start 59.86 58.64) (end 62.98 61.76) (width 1) (layer "F.Cu") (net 1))
 (segment (start 25.70164 41.71164) (end 25.70164 51.6593) (width 0.25) (layer "F.Cu") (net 1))
 (segment (start 74.89 23.5225) (end 72.0225 23.5225) (width 0.5) (layer "F.Cu") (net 1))
 (segment (start 75.5 58.77) (end 72.51 61.76) (width 0.5) (layer "F.Cu") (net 1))
 (segment (start 66.96 36.5675) (end 66.9475 36.58) (width 0.5) (layer "F.Cu") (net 1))
 (segment (start 75.34 21.25) (end 82.25 21.25) (width 0.5) (layer "F.Cu") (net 1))
 (segment (start 59.86 53.25) (end 59.86 58.64) (width 1) (layer "F.Cu") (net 1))
 (segment (start 75.5 47.35) (end 75.5 49.1) (width 0.5) (layer "F.Cu") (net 1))
 (segment (start 71.43 26.03) (end 67.45 26.03) (width 0.5) (layer "F.Cu") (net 1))
 (segment (start 24.50164 38.5093) (end 24.50164 40.51164) (width 0.25) (layer "F.Cu") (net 1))
 (segment (start 75.5 49.1) (end 75.5 58.77) (width 0.5) (layer "F.Cu") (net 1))
 (segment (start 72.0225 23.5225) (end 71.93 23.43) (width 0.5) (layer "F.Cu") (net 1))
 (via (at 81.49 40.09) (size 0.8) (drill 0.4) (layers "F.Cu" "B.Cu") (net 1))
 (segment (start 79.83 31.18) (end 79.83 23.67) (width 0.5) (layer "B.Cu") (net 1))
 (segment (start 39.24 66.24) (end 42.09 66.24) (width 0.5) (layer "B.Cu") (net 1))
 (segment (start 79.52 56.24) (end 73.98 61.78) (width 0.5) (layer "B.Cu") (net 1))
 (segment (start 86.79 56.24) (end 79.52 56.24) (width 0.5) (layer "B.Cu") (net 1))
 (segment (start 42.09 66.24) (end 42.115 66.265) (width 0.5) (layer "B.Cu") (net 1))
 (segment (start 73.96 61.76) (end 69.48 61.76) (width 0.5) (layer "B.Cu") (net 1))
 (segment (start 79.83 23.67) (end 82.25 21.25) (width 0.5) (layer "B.Cu") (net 1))
 (segment (start 81.49 40.09) (end 81.49 32.84) (width 0.5) (layer "B.Cu") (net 1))
 (segment (start 34.75 61.75) (end 39.24 66.24) (width 0.5) (layer "B.Cu") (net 1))
 (segment (start 73.98 61.78) (end 73.96 61.76) (width 0.5) (layer "B.Cu") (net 1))
 (segment (start 81.49 32.84) (end 79.83 31.18) (width 0.5) (layer "B.Cu") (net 1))
 (segment (start 34.75 61.75) (end 28.25 61.75) (width 0.5) (layer "B.Cu") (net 1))
 (segment (start 68.9975 36.58) (end 68.9975 37.3625) (width 0.5) (layer "F.Cu") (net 2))
 (segment (start 68.9975 37.3625) (end 66.99 39.37) (width 0.5) (layer "F.Cu") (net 2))
 (segment (start 66.99 39.37) (end 66.99 40.3) (width 0.5) (layer "F.Cu") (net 2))
 (segment (start 69.48 66.26) (end 62.98 66.26) (width 0.5) (layer "F.Cu") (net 8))
 (segment (start 76.3 63.86) (end 73.9 66.26) (width 0.5) (layer "F.Cu") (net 8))
 (segment (start 86.79 63.86) (end 81.5 63.86) (width 0.5) (layer "F.Cu") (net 8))
 (segment (start 81.5 63.86) (end 81.5 49.1) (width 0.5) (layer "F.Cu") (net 8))
 (segment (start 86.79 63.86) (end 76.3 63.86) (width 0.5) (layer "F.Cu") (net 8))
 (segment (start 73.9 66.26) (end 69.48 66.26) (width 0.5) (layer "F.Cu") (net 8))
 (segment (start 89.5 51.41) (end 90.89 52.8) (width 0.5) (layer "F.Cu") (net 9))
 (segment (start 89.5 49.1) (end 89.5 51.41) (width 0.5) (layer "F.Cu") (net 9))
 (segment (start 90.89 52.8) (end 90.89 59.74) (width 0.5) (layer "F.Cu") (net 9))
 (segment (start 90.89 59.74) (end 89.31 61.32) (width 0.5) (layer "F.Cu") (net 9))
 (segment (start 89.31 61.32) (end 86.79 61.32) (width 0.5) (layer "F.Cu") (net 9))
 (segment (start 88.51 58.78) (end 86.79 58.78) (width 0.5) (layer "F.Cu") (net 10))
 (segment (start 89.5 53.91) (end 89.5 57.79) (width 0.5) (layer "F.Cu") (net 10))
 (segment (start 89.5 57.79) (end 88.51 58.78) (width 0.5) (layer "F.Cu") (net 10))
 (segment (start 87.5 49.1) (end 87.5 51.91) (width 0.5) (layer "F.Cu") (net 10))
 (segment (start 87.5 51.91) (end 89.5 53.91) (width 0.5) (layer "F.Cu") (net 10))
 (segment (start 29.50164 53.75164) (end 30.07 54.32) (width 0.5) (layer "F.Cu") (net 30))
 (segment (start 79.5 33.9) (end 79.5 36.46) (width 0.5) (layer "F.Cu") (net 30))
 (segment (start 37.165 58.645) (end 42.115 58.645) (width 0.5) (layer "F.Cu") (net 30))
 (segment (start 32.84 54.32) (end 37.165 58.645) (width 0.5) (layer "F.Cu") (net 30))
 (segment (start 79.5 36.46) (end 79.51 36.47) (width 0.5) (layer "F.Cu") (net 30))
 (segment (start 29.50164 51.6693) (end 29.50164 53.75164) (width 0.5) (layer "F.Cu") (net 30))
 (segment (start 30.07 54.32) (end 32.84 54.32) (width 0.5) (layer "F.Cu") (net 30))
 (via (at 79.51 36.47) (size 0.8) (drill 0.4) (layers "F.Cu" "B.Cu") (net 30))
 (segment (start 53.76 49.15) (end 44.265 58.645) (width 0.5) (layer "B.Cu") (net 30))
 (segment (start 79.51 36.47) (end 79.51 47.96) (width 0.5) (layer "B.Cu") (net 30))
 (segment (start 44.265 58.645) (end 42.115 58.645) (width 0.5) (layer "B.Cu") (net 30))
 (segment (start 79.51 47.96) (end 78.32 49.15) (width 0.5) (layer "B.Cu") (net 30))
 (segment (start 78.32 49.15) (end 53.76 49.15) (width 0.5) (layer "B.Cu") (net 30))
 (segment (start 28.23164 51.6593) (end 28.23164 54.46164) (width 0.5) (layer "F.Cu") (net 31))
 (segment (start 32.19 55.57) (end 37.805 61.185) (width 0.5) (layer "F.Cu") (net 31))
 (segment (start 37.805 61.185) (end 42.115 61.185) (width 0.5) (layer "F.Cu") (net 31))
 (segment (start 28.23164 54.46164) (end 29.34 55.57) (width 0.5) (layer "F.Cu") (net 31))
 (segment (start 83.5 49.1) (end 83.5 46.92) (width 0.5) (layer "F.Cu") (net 31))
 (segment (start 29.34 55.57) (end 32.19 55.57) (width 0.5) (layer "F.Cu") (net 31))
 (via (at 83.5 46.92) (size 0.8) (drill 0.4) (layers "F.Cu" "B.Cu") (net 31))
 (segment (start 48.9 56.75) (end 44.465 61.185) (width 0.5) (layer "B.Cu") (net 31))
 (segment (start 73.67 56.75) (end 48.9 56.75) (width 0.5) (layer "B.Cu") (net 31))
 (segment (start 44.465 61.185) (end 42.115 61.185) (width 0.5) (layer "B.Cu") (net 31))
 (segment (start 83.5 46.92) (end 73.67 56.75) (width 0.5) (layer "B.Cu") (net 31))
 (segment (start 25.77164 40.44164) (end 25.77164 38.5093) (width 0.5) (layer "F.Cu") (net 6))
 (segment (start 28.25 66.25) (end 31.35 66.25) (width 0.5) (layer "F.Cu") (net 6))
 (segment (start 31.35 66.25) (end 34.75 66.25) (width 0.5) (layer "F.Cu") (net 6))
 (segment (start 37.275 63.725) (end 34.75 66.25) (width 0.5) (layer "F.Cu") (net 6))
 (segment (start 28.98 57.3) (end 30.11 57.3) (width 0.5) (layer "F.Cu") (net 6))
 (segment (start 25.79 40.46) (end 25.77164 40.44164) (width 0.5) (layer "F.Cu") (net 6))
 (segment (start 85.5 49.1) (end 85.5 47.07) (width 0.5) (layer "F.Cu") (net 6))
 (segment (start 85.5 47.07) (end 85.53 47.04) (width 0.5) (layer "F.Cu") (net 6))
 (segment (start 31.35 58.54) (end 31.35 66.25) (width 0.5) (layer "F.Cu") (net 6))
 (segment (start 30.11 57.3) (end 31.35 58.54) (width 0.5) (layer "F.Cu") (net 6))
 (segment (start 42.115 63.725) (end 37.275 63.725) (width 0.5) (layer "F.Cu") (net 6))
 (via (at 28.98 57.3) (size 0.8) (drill 0.4) (layers "F.Cu" "B.Cu") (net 6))
 (via (at 25.79 40.46) (size 0.8) (drill 0.4) (layers "F.Cu" "B.Cu") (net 6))
 (via (at 85.53 47.04) (size 0.8) (drill 0.4) (layers "F.Cu" "B.Cu") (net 6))
 (segment (start 25.8 40.46) (end 28.98 43.64) (width 0.5) (layer "B.Cu") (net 6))
 (segment (start 25.79 40.46) (end 25.8 40.46) (width 0.5) (layer "B.Cu") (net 6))
 (segment (start 44.655 63.725) (end 42.115 63.725) (width 0.5) (layer "B.Cu") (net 6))
 (segment (start 49.98 58.4) (end 44.655 63.725) (width 0.5) (layer "B.Cu") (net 6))
 (segment (start 28.98 43.64) (end 28.98 57.3) (width 0.5) (layer "B.Cu") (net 6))
 (segment (start 85.53 47.04) (end 74.17 58.4) (width 0.5) (layer "B.Cu") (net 6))
 (segment (start 74.17 58.4) (end 49.98 58.4) (width 0.5) (layer "B.Cu") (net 6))
 (segment (start 85.5 33.9) (end 85.5 28.91) (width 0.5) (layer "F.Cu") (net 33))
 (segment (start 85.5 28.91) (end 85.52 28.89) (width 0.5) (layer "F.Cu") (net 33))
 (segment (start 89.5 29.71) (end 89.5 33.9) (width 0.5) (layer "F.Cu") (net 34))
 (segment (start 80.04 23.54) (end 82.25 25.75) (width 0.5) (layer "F.Cu") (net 34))
 (segment (start 88.75 28.96) (end 89.5 29.71) (width 0.5) (layer "F.Cu") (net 34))
 (segment (start 77.53 23.54) (end 80.04 23.54) (width 0.5) (layer "F.Cu") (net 34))
 (segment (start 88.75 25.75) (end 88.75 28.96) (width 0.5) (layer "F.Cu") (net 34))
 (segment (start 30.87 38.54766) (end 30.84164 38.5193) (width 0.5) (layer "F.Cu") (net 14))
 (segment (start 77.5 36.33) (end 77.46 36.37) (width 0.5) (layer "F.Cu") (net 14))
 (segment (start 77.5 33.9) (end 77.5 36.33) (width 0.5) (layer "F.Cu") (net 14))
 (segment (start 30.87 40.84) (end 30.87 38.54766) (width 0.5) (layer "F.Cu") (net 14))
 (via (at 30.87 40.84) (size 0.8) (drill 0.4) (layers "F.Cu" "B.Cu") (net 14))
 (via (at 77.46 36.37) (size 0.8) (drill 0.4) (layers "F.Cu" "B.Cu") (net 14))
 (segment (start 75.51 45.12) (end 77.46 43.17) (width 0.5) (layer "B.Cu") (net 14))
 (segment (start 30.87 40.84) (end 35.15 45.12) (width 0.5) (layer "B.Cu") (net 14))
 (segment (start 35.15 45.12) (end 75.51 45.12) (width 0.5) (layer "B.Cu") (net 14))
 (segment (start 77.46 43.17) (end 77.46 36.37) (width 0.5) (layer "B.Cu") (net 14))
 (segment (start 77.5 49.1) (end 77.5 46.89) (width 0.5) (layer "F.Cu") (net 13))
 (segment (start 29.58 40.85) (end 29.58 38.52766) (width 0.5) (layer "F.Cu") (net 13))
 (segment (start 29.58 38.52766) (end 29.57164 38.5193) (width 0.5) (layer "F.Cu") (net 13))
 (via (at 29.58 40.85) (size 0.8) (drill 0.4) (layers "F.Cu" "B.Cu") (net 13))
 (via (at 77.5 46.89) (size 0.8) (drill 0.4) (layers "F.Cu" "B.Cu") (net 13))
 (segment (start 29.58 42.21) (end 29.58 40.85) (width 0.5) (layer "B.Cu") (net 13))
 (segment (start 77.5 46.89) (end 34.26 46.89) (width 0.5) (layer "B.Cu") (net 13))
 (segment (start 34.26 46.89) (end 29.58 42.21) (width 0.5) (layer "B.Cu") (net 13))
 (segment (start 63.31 23.43) (end 47 39.74) (width 0.5) (layer "F.Cu") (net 5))
 (segment (start 67.33 23.43) (end 63.31 23.43) (width 0.5) (layer "F.Cu") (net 5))
 (segment (start 67.3 23.4) (end 67.33 23.43) (width 0.5) (layer "F.Cu") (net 5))
 (segment (start 67.3 19.84) (end 67.3 23.4) (width 0.5) (layer "F.Cu") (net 5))
 (segment (start 47 39.74) (end 47 50.71) (width 0.5) (layer "F.Cu") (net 5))
 (segment (start 57.2 21.31) (end 57.2 20.16) (width 1) (layer "B.Cu") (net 3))
 (segment (start 41.21 19.02) (end 39.37 20.86) (width 1) (layer "B.Cu") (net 3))
 (segment (start 57.2 20.16) (end 56.06 19.02) (width 1) (layer "B.Cu") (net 3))
 (segment (start 56.06 19.02) (end 41.21 19.02) (width 1) (layer "B.Cu") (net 3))
 (segment (start 30.51 20.94) (end 33.8 24.23) (width 1) (layer "B.Cu") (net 4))
 (segment (start 49.28 24.23) (end 52.2 21.31) (width 1) (layer "B.Cu") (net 4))
 (segment (start 33.8 24.23) (end 49.28 24.23) (width 1) (layer "B.Cu") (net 4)))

